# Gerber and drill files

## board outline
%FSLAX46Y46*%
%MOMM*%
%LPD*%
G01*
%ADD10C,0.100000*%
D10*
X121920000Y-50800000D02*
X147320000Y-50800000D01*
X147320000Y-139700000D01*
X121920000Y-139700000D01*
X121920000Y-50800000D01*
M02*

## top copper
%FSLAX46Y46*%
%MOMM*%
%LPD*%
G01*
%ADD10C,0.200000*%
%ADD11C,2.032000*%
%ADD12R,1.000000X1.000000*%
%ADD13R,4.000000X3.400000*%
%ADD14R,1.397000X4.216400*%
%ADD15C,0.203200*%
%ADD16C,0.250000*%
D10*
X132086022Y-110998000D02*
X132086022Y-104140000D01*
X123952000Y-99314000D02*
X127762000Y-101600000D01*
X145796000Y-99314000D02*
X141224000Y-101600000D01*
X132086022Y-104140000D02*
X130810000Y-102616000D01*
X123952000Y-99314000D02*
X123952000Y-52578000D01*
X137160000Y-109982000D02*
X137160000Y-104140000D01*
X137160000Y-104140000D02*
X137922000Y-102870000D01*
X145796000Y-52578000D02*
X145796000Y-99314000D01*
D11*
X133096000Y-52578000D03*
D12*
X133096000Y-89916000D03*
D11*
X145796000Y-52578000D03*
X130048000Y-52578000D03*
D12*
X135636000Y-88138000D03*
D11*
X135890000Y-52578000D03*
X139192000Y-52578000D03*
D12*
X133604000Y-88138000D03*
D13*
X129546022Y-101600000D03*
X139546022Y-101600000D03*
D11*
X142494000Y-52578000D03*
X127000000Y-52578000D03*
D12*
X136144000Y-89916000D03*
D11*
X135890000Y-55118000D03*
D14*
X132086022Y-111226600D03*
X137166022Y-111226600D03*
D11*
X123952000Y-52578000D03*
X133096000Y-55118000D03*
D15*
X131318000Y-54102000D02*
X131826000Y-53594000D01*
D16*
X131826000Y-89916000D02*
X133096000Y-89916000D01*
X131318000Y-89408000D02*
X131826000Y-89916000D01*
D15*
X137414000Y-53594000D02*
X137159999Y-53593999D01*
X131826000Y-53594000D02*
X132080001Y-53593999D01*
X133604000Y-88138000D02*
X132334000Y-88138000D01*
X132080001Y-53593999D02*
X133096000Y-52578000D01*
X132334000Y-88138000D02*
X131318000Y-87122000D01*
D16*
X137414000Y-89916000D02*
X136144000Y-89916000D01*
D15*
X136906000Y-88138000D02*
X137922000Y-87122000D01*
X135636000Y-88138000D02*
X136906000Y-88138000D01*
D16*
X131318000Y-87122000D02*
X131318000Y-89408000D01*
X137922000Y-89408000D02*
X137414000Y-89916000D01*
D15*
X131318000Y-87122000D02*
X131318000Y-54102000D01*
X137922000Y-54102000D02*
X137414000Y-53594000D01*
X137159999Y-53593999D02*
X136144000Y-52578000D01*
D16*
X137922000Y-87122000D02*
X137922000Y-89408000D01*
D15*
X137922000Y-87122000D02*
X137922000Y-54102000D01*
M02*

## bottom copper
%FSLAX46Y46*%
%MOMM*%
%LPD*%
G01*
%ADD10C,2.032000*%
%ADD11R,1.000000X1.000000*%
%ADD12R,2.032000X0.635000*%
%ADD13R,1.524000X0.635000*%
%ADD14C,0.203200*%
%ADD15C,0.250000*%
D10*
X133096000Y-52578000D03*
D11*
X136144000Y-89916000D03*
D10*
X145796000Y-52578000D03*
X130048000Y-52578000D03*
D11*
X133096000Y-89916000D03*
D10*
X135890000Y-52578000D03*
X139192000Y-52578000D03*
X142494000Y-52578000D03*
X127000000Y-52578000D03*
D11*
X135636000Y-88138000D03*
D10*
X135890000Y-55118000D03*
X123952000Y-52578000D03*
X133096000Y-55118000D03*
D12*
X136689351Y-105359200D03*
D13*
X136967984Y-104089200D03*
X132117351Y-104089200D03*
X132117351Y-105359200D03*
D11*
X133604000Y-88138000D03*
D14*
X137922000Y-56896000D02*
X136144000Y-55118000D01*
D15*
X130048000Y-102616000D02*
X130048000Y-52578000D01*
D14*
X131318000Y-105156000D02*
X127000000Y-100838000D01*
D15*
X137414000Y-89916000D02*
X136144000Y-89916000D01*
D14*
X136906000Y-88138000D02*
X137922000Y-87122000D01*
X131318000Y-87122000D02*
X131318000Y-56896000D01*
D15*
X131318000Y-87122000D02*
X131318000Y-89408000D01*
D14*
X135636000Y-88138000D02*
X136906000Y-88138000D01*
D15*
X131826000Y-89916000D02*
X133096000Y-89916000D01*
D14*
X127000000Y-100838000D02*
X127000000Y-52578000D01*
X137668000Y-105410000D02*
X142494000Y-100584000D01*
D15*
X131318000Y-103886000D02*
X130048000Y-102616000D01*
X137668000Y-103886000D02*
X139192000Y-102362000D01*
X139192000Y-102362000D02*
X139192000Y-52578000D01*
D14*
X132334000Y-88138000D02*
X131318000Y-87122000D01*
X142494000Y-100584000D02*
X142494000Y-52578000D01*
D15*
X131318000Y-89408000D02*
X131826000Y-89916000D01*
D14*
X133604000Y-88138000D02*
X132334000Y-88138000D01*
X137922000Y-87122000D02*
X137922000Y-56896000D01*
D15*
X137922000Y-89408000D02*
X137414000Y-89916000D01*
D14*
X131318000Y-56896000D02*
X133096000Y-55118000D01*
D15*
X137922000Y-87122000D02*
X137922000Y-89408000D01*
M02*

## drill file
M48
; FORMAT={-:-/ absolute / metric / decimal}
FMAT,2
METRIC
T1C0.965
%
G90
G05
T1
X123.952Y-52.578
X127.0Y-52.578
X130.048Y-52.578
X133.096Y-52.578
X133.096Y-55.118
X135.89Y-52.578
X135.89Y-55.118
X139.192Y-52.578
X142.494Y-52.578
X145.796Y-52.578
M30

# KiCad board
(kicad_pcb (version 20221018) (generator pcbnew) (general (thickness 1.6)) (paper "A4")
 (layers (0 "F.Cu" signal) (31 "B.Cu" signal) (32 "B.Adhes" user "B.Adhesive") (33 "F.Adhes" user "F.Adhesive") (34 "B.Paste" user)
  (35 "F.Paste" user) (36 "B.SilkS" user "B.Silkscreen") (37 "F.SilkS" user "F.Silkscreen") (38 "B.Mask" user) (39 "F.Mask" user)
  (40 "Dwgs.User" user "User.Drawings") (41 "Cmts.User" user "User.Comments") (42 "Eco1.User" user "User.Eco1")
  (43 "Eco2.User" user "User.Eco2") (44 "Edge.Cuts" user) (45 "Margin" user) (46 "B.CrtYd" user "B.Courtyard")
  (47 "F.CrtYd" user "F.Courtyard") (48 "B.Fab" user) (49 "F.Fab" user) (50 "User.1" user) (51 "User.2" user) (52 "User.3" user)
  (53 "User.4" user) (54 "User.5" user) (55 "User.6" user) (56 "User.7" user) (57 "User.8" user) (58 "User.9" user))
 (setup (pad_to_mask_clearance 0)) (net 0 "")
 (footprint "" (layer "F.Cu") (at 133.096 52.578)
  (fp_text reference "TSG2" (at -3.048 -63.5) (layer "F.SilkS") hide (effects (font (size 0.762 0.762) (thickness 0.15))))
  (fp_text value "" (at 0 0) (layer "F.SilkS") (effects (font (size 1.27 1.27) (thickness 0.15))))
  (pad "1" thru_hole circle (at 0 0) (size 2.032 2.032) (drill 0.9652) (layers "*.Cu" "*.Mask")))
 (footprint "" (layer "F.Cu") (at 133.096 89.916)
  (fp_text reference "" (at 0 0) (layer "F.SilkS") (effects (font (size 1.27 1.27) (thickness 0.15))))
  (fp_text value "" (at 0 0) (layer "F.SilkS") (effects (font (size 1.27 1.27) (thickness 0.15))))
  (pad "1" smd rect (at 0 0) (size 1 1) (layers "F.Cu" "F.Mask")))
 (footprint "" (layer "F.Cu") (at 136.144 89.916)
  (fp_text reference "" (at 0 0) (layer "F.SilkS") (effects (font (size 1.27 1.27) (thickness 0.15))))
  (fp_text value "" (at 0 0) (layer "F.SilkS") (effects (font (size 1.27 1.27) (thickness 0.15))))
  (pad "1" smd rect (at 0 0 180) (size 1 1) (layers "B.Cu" "B.Mask")))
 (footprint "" (layer "F.Cu") (at 145.796 66.04)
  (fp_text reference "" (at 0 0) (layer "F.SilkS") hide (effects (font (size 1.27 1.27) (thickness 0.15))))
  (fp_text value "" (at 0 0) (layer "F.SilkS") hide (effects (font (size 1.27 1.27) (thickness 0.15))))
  (pad "1" thru_hole circle (at 0 -13.462) (size 2.032 2.032) (drill 0.9652) (layers "*.Cu" "*.Mask")))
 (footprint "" (layer "F.Cu") (at 130.048 66.04)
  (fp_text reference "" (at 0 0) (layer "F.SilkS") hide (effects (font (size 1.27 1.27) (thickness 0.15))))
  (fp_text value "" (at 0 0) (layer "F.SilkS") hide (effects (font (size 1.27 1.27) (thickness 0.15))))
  (pad "1" thru_hole circle (at 0 -13.462) (size 2.032 2.032) (drill 0.9652) (layers "*.Cu" "*.Mask")))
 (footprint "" (layer "F.Cu") (at 133.096 89.916)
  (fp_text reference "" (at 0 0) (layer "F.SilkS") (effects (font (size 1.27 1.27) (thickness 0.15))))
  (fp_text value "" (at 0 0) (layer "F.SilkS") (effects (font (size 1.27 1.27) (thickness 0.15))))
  (pad "1" smd rect (at 0 0 180) (size 1 1) (layers "B.Cu" "B.Mask")))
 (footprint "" (layer "F.Cu") (at 135.636 88.138)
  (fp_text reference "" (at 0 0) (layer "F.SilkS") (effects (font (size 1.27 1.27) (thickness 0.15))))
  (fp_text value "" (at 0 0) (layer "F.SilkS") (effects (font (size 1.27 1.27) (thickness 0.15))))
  (pad "1" smd rect (at 0 0) (size 1 1) (layers "F.Cu" "F.Mask")))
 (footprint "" (layer "F.Cu") (at 135.89 52.578)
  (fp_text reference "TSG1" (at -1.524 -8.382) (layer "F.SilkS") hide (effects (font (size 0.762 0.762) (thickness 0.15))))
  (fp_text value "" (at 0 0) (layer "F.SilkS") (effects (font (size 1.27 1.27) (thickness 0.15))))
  (pad "1" thru_hole circle (at 0 0) (size 2.032 2.032) (drill 0.9652) (layers "*.Cu" "*.Mask")))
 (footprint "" (layer "F.Cu") (at 139.192 66.04)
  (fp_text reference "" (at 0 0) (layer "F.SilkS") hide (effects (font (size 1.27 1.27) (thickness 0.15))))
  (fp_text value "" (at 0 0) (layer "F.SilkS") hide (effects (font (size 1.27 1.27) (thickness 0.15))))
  (pad "1" thru_hole circle (at 0 -13.462) (size 2.032 2.032) (drill 0.9652) (layers "*.Cu" "*.Mask")))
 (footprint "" (layer "F.Cu") (at 133.604 75.438)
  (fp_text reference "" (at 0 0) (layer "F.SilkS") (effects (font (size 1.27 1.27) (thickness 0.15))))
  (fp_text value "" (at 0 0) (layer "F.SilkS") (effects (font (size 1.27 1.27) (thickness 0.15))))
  (pad "1" smd rect (at 0 12.7) (size 1 1) (layers "F.Cu" "F.Mask")))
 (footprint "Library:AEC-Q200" (layer "F.Cu") (at 134.626022 107.95)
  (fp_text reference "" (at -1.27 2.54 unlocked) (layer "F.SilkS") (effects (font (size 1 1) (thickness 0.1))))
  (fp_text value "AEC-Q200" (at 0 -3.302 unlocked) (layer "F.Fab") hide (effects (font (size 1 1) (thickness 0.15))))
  (pad "1" smd rect (at -5.08 -6.35 180) (size 4 3.4) (layers "F.Cu" "F.Mask"))
  (pad "2" smd rect (at 4.92 -6.35 180) (size 4 3.4) (layers "F.Cu" "F.Mask")))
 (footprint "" (layer "F.Cu") (at 142.494 66.04)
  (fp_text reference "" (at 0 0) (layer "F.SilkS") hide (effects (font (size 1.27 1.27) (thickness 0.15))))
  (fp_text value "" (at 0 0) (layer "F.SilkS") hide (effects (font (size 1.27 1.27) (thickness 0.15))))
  (pad "1" thru_hole circle (at 0 -13.462) (size 2.032 2.032) (drill 0.9652) (layers "*.Cu" "*.Mask")))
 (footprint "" (layer "F.Cu") (at 127 66.04)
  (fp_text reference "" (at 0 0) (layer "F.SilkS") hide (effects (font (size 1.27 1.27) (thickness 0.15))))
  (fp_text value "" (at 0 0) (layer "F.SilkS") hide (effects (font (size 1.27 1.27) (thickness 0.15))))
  (pad "1" thru_hole circle (at 0 -13.462) (size 2.032 2.032) (drill 0.9652) (layers "*.Cu" "*.Mask")))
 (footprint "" (layer "F.Cu") (at 135.636 88.138)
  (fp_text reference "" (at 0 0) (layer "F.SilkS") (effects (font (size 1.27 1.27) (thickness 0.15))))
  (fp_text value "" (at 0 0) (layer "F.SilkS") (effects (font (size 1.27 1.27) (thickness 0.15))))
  (pad "1" smd rect (at 0 0 180) (size 1 1) (layers "B.Cu" "B.Mask")))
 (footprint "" (layer "F.Cu") (at 136.144 89.916)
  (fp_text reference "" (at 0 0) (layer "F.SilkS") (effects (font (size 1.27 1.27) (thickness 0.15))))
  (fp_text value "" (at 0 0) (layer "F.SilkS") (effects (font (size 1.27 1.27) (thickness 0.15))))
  (pad "1" smd rect (at 0 0) (size 1 1) (layers "F.Cu" "F.Mask")))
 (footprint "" (layer "F.Cu") (at 135.89 55.118)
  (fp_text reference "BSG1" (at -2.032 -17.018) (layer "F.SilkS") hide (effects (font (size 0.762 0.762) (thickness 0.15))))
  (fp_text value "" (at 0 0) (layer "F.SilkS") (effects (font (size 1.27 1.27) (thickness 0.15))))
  (pad "1" thru_hole circle (at 0 0) (size 2.032 2.032) (drill 0.9652) (layers "*.Cu" "*.Mask")))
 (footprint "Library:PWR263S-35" (layer "F.Cu") (at 135.896022 112.268)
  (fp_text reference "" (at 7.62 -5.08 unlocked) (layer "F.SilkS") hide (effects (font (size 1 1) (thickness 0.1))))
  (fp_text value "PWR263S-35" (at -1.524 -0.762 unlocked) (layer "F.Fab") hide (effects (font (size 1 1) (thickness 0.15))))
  (pad "1" smd rect (at -3.81 -1.0414) (size 1.397 4.2164) (layers "F.Cu" "F.Mask"))
  (pad "2" smd rect (at 1.27 -1.0414) (size 1.397 4.2164) (layers "F.Cu" "F.Mask")))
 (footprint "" (layer "F.Cu") (at 123.952 66.04)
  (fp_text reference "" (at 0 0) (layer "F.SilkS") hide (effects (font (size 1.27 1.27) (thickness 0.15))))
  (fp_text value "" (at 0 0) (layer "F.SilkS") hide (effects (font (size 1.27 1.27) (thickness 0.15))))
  (pad "1" thru_hole circle (at 0 -13.462) (size 2.032 2.032) (drill 0.9652) (layers "*.Cu" "*.Mask")))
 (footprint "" (layer "F.Cu") (at 133.096 55.118)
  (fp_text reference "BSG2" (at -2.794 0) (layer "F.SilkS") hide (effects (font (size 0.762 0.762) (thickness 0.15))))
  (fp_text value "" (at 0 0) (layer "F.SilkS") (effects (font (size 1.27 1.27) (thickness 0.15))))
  (pad "1" thru_hole circle (at 0 0) (size 2.032 2.032) (drill 0.9652) (layers "*.Cu" "*.Mask")))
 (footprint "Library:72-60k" (layer "B.Cu") (at 132.879351 109.1692 180)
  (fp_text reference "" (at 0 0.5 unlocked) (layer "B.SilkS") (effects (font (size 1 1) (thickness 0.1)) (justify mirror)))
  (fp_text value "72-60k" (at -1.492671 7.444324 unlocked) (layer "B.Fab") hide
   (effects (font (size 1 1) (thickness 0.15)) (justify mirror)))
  (pad "1" smd rect (at -3.81 3.81) (size 2.032 0.635) (layers "B.Cu" "B.Mask"))
  (pad "2" smd rect (at -4.088633 5.08) (size 1.524 0.635) (layers "B.Cu" "B.Mask"))
  (pad "3" smd rect (at 0.762 5.08) (size 1.524 0.635) (layers "B.Cu" "B.Mask"))
  (pad "4" smd rect (at 0.762 3.81) (size 1.524 0.635) (layers "B.Cu" "B.Mask")))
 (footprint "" (layer "B.Cu") (at 133.604 75.438 180)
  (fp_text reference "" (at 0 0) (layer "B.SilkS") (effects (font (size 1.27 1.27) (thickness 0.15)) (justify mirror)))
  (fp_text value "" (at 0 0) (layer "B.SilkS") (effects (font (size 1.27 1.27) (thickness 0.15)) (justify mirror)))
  (pad "1" smd rect (at 0 -12.7 180) (size 1 1) (layers "B.Cu" "B.Mask")))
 (gr_line (start 132.086022 110.998) (end 132.086022 104.14) (stroke (width 0.2) (type default)) (layer "F.Cu"))
 (gr_line (start 123.952 99.314) (end 127.762 101.6) (stroke (width 0.2) (type default)) (layer "F.Cu"))
 (gr_line (start 145.796 99.314) (end 141.224 101.6) (stroke (width 0.2) (type default)) (layer "F.Cu"))
 (gr_line (start 132.086022 104.14) (end 130.81 102.616) (stroke (width 0.2) (type default)) (layer "F.Cu"))
 (gr_line (start 123.952 99.314) (end 123.952 52.578) (stroke (width 0.2) (type default)) (layer "F.Cu"))
 (gr_line (start 137.16 109.982) (end 137.16 104.14) (stroke (width 0.2) (type default)) (layer "F.Cu"))
 (gr_line (start 137.16 104.14) (end 137.922 102.87) (stroke (width 0.2) (type default)) (layer "F.Cu"))
 (gr_line (start 145.796 52.578) (end 145.796 99.314) (stroke (width 0.2) (type default)) (layer "F.Cu"))
 (gr_rect (start 121.92 50.8) (end 147.32 139.7) (stroke (width 0.1) (type default)) (fill none) (layer "Edge.Cuts"))
 (segment (start 131.318 54.102) (end 131.826 53.594) (width 0.2032) (layer "F.Cu") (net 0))
 (segment (start 131.826 89.916) (end 133.096 89.916) (width 0.25) (layer "F.Cu") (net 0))
 (segment (start 131.318 89.408) (end 131.826 89.916) (width 0.25) (layer "F.Cu") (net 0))
 (segment (start 137.414 53.594) (end 137.159999 53.593999) (width 0.2032) (layer "F.Cu") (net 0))
 (segment (start 131.826 53.594) (end 132.080001 53.593999) (width 0.2032) (layer "F.Cu") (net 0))
 (segment (start 133.604 88.138) (end 132.334 88.138) (width 0.2032) (layer "F.Cu") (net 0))
 (segment (start 132.080001 53.593999) (end 133.096 52.578) (width 0.2032) (layer "F.Cu") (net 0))
 (segment (start 132.334 88.138) (end 131.318 87.122) (width 0.2032) (layer "F.Cu") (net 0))
 (segment (start 137.414 89.916) (end 136.144 89.916) (width 0.25) (layer "F.Cu") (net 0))
 (segment (start 136.906 88.138) (end 137.922 87.122) (width 0.2032) (layer "F.Cu") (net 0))
 (segment (start 135.636 88.138) (end 136.906 88.138) (width 0.2032) (layer "F.Cu") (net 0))
 (segment (start 131.318 87.122) (end 131.318 89.408) (width 0.25) (layer "F.Cu") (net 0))
 (segment (start 137.922 89.408) (end 137.414 89.916) (width 0.25) (layer "F.Cu") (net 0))
 (segment (start 131.318 87.122) (end 131.318 54.102) (width 0.2032) (layer "F.Cu") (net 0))
 (segment (start 137.922 54.102) (end 137.414 53.594) (width 0.2032) (layer "F.Cu") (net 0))
 (segment (start 137.159999 53.593999) (end 136.144 52.578) (width 0.2032) (layer "F.Cu") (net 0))
 (segment (start 137.922 87.122) (end 137.922 89.408) (width 0.25) (layer "F.Cu") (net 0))
 (segment (start 137.922 87.122) (end 137.922 54.102) (width 0.2032) (layer "F.Cu") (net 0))
 (segment (start 137.922 56.896) (end 136.144 55.118) (width 0.2032) (layer "B.Cu") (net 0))
 (segment (start 130.048 102.616) (end 130.048 52.578) (width 0.25) (layer "B.Cu") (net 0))
 (segment (start 131.318 105.156) (end 127 100.838) (width 0.2032) (layer "B.Cu") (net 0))
 (segment (start 137.414 89.916) (end 136.144 89.916) (width 0.25) (layer "B.Cu") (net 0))
 (segment (start 136.906 88.138) (end 137.922 87.122) (width 0.2032) (layer "B.Cu") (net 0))
 (segment (start 131.318 87.122) (end 131.318 56.896) (width 0.2032) (layer "B.Cu") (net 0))
 (segment (start 131.318 87.122) (end 131.318 89.408) (width 0.25) (layer "B.Cu") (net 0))
 (segment (start 135.636 88.138) (end 136.906 88.138) (width 0.2032) (layer "B.Cu") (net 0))
 (segment (start 131.826 89.916) (end 133.096 89.916) (width 0.25) (layer "B.Cu") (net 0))
 (segment (start 127 100.838) (end 127 52.578) (width 0.2032) (layer "B.Cu") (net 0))
 (segment (start 137.668 105.41) (end 142.494 100.584) (width 0.2032) (layer "B.Cu") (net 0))
 (segment (start 131.318 103.886) (end 130.048 102.616) (width 0.25) (layer "B.Cu") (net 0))
 (segment (start 137.668 103.886) (end 139.192 102.362) (width 0.25) (layer "B.Cu") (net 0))
 (segment (start 139.192 102.362) (end 139.192 52.578) (width 0.25) (layer "B.Cu") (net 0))
 (segment (start 132.334 88.138) (end 131.318 87.122) (width 0.2032) (layer "B.Cu") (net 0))
 (segment (start 142.494 100.584) (end 142.494 52.578) (width 0.2032) (layer "B.Cu") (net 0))
 (segment (start 131.318 89.408) (end 131.826 89.916) (width 0.25) (layer "B.Cu") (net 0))
 (segment (start 133.604 88.138) (end 132.334 88.138) (width 0.2032) (layer "B.Cu") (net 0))
 (segment (start 137.922 87.122) (end 137.922 56.896) (width 0.2032) (layer "B.Cu") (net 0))
 (segment (start 137.922 89.408) (end 137.414 89.916) (width 0.25) (layer "B.Cu") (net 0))
 (segment (start 131.318 56.896) (end 133.096 55.118) (width 0.2032) (layer "B.Cu") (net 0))
 (segment (start 137.922 87.122) (end 137.922 89.408) (width 0.25) (layer "B.Cu") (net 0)))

